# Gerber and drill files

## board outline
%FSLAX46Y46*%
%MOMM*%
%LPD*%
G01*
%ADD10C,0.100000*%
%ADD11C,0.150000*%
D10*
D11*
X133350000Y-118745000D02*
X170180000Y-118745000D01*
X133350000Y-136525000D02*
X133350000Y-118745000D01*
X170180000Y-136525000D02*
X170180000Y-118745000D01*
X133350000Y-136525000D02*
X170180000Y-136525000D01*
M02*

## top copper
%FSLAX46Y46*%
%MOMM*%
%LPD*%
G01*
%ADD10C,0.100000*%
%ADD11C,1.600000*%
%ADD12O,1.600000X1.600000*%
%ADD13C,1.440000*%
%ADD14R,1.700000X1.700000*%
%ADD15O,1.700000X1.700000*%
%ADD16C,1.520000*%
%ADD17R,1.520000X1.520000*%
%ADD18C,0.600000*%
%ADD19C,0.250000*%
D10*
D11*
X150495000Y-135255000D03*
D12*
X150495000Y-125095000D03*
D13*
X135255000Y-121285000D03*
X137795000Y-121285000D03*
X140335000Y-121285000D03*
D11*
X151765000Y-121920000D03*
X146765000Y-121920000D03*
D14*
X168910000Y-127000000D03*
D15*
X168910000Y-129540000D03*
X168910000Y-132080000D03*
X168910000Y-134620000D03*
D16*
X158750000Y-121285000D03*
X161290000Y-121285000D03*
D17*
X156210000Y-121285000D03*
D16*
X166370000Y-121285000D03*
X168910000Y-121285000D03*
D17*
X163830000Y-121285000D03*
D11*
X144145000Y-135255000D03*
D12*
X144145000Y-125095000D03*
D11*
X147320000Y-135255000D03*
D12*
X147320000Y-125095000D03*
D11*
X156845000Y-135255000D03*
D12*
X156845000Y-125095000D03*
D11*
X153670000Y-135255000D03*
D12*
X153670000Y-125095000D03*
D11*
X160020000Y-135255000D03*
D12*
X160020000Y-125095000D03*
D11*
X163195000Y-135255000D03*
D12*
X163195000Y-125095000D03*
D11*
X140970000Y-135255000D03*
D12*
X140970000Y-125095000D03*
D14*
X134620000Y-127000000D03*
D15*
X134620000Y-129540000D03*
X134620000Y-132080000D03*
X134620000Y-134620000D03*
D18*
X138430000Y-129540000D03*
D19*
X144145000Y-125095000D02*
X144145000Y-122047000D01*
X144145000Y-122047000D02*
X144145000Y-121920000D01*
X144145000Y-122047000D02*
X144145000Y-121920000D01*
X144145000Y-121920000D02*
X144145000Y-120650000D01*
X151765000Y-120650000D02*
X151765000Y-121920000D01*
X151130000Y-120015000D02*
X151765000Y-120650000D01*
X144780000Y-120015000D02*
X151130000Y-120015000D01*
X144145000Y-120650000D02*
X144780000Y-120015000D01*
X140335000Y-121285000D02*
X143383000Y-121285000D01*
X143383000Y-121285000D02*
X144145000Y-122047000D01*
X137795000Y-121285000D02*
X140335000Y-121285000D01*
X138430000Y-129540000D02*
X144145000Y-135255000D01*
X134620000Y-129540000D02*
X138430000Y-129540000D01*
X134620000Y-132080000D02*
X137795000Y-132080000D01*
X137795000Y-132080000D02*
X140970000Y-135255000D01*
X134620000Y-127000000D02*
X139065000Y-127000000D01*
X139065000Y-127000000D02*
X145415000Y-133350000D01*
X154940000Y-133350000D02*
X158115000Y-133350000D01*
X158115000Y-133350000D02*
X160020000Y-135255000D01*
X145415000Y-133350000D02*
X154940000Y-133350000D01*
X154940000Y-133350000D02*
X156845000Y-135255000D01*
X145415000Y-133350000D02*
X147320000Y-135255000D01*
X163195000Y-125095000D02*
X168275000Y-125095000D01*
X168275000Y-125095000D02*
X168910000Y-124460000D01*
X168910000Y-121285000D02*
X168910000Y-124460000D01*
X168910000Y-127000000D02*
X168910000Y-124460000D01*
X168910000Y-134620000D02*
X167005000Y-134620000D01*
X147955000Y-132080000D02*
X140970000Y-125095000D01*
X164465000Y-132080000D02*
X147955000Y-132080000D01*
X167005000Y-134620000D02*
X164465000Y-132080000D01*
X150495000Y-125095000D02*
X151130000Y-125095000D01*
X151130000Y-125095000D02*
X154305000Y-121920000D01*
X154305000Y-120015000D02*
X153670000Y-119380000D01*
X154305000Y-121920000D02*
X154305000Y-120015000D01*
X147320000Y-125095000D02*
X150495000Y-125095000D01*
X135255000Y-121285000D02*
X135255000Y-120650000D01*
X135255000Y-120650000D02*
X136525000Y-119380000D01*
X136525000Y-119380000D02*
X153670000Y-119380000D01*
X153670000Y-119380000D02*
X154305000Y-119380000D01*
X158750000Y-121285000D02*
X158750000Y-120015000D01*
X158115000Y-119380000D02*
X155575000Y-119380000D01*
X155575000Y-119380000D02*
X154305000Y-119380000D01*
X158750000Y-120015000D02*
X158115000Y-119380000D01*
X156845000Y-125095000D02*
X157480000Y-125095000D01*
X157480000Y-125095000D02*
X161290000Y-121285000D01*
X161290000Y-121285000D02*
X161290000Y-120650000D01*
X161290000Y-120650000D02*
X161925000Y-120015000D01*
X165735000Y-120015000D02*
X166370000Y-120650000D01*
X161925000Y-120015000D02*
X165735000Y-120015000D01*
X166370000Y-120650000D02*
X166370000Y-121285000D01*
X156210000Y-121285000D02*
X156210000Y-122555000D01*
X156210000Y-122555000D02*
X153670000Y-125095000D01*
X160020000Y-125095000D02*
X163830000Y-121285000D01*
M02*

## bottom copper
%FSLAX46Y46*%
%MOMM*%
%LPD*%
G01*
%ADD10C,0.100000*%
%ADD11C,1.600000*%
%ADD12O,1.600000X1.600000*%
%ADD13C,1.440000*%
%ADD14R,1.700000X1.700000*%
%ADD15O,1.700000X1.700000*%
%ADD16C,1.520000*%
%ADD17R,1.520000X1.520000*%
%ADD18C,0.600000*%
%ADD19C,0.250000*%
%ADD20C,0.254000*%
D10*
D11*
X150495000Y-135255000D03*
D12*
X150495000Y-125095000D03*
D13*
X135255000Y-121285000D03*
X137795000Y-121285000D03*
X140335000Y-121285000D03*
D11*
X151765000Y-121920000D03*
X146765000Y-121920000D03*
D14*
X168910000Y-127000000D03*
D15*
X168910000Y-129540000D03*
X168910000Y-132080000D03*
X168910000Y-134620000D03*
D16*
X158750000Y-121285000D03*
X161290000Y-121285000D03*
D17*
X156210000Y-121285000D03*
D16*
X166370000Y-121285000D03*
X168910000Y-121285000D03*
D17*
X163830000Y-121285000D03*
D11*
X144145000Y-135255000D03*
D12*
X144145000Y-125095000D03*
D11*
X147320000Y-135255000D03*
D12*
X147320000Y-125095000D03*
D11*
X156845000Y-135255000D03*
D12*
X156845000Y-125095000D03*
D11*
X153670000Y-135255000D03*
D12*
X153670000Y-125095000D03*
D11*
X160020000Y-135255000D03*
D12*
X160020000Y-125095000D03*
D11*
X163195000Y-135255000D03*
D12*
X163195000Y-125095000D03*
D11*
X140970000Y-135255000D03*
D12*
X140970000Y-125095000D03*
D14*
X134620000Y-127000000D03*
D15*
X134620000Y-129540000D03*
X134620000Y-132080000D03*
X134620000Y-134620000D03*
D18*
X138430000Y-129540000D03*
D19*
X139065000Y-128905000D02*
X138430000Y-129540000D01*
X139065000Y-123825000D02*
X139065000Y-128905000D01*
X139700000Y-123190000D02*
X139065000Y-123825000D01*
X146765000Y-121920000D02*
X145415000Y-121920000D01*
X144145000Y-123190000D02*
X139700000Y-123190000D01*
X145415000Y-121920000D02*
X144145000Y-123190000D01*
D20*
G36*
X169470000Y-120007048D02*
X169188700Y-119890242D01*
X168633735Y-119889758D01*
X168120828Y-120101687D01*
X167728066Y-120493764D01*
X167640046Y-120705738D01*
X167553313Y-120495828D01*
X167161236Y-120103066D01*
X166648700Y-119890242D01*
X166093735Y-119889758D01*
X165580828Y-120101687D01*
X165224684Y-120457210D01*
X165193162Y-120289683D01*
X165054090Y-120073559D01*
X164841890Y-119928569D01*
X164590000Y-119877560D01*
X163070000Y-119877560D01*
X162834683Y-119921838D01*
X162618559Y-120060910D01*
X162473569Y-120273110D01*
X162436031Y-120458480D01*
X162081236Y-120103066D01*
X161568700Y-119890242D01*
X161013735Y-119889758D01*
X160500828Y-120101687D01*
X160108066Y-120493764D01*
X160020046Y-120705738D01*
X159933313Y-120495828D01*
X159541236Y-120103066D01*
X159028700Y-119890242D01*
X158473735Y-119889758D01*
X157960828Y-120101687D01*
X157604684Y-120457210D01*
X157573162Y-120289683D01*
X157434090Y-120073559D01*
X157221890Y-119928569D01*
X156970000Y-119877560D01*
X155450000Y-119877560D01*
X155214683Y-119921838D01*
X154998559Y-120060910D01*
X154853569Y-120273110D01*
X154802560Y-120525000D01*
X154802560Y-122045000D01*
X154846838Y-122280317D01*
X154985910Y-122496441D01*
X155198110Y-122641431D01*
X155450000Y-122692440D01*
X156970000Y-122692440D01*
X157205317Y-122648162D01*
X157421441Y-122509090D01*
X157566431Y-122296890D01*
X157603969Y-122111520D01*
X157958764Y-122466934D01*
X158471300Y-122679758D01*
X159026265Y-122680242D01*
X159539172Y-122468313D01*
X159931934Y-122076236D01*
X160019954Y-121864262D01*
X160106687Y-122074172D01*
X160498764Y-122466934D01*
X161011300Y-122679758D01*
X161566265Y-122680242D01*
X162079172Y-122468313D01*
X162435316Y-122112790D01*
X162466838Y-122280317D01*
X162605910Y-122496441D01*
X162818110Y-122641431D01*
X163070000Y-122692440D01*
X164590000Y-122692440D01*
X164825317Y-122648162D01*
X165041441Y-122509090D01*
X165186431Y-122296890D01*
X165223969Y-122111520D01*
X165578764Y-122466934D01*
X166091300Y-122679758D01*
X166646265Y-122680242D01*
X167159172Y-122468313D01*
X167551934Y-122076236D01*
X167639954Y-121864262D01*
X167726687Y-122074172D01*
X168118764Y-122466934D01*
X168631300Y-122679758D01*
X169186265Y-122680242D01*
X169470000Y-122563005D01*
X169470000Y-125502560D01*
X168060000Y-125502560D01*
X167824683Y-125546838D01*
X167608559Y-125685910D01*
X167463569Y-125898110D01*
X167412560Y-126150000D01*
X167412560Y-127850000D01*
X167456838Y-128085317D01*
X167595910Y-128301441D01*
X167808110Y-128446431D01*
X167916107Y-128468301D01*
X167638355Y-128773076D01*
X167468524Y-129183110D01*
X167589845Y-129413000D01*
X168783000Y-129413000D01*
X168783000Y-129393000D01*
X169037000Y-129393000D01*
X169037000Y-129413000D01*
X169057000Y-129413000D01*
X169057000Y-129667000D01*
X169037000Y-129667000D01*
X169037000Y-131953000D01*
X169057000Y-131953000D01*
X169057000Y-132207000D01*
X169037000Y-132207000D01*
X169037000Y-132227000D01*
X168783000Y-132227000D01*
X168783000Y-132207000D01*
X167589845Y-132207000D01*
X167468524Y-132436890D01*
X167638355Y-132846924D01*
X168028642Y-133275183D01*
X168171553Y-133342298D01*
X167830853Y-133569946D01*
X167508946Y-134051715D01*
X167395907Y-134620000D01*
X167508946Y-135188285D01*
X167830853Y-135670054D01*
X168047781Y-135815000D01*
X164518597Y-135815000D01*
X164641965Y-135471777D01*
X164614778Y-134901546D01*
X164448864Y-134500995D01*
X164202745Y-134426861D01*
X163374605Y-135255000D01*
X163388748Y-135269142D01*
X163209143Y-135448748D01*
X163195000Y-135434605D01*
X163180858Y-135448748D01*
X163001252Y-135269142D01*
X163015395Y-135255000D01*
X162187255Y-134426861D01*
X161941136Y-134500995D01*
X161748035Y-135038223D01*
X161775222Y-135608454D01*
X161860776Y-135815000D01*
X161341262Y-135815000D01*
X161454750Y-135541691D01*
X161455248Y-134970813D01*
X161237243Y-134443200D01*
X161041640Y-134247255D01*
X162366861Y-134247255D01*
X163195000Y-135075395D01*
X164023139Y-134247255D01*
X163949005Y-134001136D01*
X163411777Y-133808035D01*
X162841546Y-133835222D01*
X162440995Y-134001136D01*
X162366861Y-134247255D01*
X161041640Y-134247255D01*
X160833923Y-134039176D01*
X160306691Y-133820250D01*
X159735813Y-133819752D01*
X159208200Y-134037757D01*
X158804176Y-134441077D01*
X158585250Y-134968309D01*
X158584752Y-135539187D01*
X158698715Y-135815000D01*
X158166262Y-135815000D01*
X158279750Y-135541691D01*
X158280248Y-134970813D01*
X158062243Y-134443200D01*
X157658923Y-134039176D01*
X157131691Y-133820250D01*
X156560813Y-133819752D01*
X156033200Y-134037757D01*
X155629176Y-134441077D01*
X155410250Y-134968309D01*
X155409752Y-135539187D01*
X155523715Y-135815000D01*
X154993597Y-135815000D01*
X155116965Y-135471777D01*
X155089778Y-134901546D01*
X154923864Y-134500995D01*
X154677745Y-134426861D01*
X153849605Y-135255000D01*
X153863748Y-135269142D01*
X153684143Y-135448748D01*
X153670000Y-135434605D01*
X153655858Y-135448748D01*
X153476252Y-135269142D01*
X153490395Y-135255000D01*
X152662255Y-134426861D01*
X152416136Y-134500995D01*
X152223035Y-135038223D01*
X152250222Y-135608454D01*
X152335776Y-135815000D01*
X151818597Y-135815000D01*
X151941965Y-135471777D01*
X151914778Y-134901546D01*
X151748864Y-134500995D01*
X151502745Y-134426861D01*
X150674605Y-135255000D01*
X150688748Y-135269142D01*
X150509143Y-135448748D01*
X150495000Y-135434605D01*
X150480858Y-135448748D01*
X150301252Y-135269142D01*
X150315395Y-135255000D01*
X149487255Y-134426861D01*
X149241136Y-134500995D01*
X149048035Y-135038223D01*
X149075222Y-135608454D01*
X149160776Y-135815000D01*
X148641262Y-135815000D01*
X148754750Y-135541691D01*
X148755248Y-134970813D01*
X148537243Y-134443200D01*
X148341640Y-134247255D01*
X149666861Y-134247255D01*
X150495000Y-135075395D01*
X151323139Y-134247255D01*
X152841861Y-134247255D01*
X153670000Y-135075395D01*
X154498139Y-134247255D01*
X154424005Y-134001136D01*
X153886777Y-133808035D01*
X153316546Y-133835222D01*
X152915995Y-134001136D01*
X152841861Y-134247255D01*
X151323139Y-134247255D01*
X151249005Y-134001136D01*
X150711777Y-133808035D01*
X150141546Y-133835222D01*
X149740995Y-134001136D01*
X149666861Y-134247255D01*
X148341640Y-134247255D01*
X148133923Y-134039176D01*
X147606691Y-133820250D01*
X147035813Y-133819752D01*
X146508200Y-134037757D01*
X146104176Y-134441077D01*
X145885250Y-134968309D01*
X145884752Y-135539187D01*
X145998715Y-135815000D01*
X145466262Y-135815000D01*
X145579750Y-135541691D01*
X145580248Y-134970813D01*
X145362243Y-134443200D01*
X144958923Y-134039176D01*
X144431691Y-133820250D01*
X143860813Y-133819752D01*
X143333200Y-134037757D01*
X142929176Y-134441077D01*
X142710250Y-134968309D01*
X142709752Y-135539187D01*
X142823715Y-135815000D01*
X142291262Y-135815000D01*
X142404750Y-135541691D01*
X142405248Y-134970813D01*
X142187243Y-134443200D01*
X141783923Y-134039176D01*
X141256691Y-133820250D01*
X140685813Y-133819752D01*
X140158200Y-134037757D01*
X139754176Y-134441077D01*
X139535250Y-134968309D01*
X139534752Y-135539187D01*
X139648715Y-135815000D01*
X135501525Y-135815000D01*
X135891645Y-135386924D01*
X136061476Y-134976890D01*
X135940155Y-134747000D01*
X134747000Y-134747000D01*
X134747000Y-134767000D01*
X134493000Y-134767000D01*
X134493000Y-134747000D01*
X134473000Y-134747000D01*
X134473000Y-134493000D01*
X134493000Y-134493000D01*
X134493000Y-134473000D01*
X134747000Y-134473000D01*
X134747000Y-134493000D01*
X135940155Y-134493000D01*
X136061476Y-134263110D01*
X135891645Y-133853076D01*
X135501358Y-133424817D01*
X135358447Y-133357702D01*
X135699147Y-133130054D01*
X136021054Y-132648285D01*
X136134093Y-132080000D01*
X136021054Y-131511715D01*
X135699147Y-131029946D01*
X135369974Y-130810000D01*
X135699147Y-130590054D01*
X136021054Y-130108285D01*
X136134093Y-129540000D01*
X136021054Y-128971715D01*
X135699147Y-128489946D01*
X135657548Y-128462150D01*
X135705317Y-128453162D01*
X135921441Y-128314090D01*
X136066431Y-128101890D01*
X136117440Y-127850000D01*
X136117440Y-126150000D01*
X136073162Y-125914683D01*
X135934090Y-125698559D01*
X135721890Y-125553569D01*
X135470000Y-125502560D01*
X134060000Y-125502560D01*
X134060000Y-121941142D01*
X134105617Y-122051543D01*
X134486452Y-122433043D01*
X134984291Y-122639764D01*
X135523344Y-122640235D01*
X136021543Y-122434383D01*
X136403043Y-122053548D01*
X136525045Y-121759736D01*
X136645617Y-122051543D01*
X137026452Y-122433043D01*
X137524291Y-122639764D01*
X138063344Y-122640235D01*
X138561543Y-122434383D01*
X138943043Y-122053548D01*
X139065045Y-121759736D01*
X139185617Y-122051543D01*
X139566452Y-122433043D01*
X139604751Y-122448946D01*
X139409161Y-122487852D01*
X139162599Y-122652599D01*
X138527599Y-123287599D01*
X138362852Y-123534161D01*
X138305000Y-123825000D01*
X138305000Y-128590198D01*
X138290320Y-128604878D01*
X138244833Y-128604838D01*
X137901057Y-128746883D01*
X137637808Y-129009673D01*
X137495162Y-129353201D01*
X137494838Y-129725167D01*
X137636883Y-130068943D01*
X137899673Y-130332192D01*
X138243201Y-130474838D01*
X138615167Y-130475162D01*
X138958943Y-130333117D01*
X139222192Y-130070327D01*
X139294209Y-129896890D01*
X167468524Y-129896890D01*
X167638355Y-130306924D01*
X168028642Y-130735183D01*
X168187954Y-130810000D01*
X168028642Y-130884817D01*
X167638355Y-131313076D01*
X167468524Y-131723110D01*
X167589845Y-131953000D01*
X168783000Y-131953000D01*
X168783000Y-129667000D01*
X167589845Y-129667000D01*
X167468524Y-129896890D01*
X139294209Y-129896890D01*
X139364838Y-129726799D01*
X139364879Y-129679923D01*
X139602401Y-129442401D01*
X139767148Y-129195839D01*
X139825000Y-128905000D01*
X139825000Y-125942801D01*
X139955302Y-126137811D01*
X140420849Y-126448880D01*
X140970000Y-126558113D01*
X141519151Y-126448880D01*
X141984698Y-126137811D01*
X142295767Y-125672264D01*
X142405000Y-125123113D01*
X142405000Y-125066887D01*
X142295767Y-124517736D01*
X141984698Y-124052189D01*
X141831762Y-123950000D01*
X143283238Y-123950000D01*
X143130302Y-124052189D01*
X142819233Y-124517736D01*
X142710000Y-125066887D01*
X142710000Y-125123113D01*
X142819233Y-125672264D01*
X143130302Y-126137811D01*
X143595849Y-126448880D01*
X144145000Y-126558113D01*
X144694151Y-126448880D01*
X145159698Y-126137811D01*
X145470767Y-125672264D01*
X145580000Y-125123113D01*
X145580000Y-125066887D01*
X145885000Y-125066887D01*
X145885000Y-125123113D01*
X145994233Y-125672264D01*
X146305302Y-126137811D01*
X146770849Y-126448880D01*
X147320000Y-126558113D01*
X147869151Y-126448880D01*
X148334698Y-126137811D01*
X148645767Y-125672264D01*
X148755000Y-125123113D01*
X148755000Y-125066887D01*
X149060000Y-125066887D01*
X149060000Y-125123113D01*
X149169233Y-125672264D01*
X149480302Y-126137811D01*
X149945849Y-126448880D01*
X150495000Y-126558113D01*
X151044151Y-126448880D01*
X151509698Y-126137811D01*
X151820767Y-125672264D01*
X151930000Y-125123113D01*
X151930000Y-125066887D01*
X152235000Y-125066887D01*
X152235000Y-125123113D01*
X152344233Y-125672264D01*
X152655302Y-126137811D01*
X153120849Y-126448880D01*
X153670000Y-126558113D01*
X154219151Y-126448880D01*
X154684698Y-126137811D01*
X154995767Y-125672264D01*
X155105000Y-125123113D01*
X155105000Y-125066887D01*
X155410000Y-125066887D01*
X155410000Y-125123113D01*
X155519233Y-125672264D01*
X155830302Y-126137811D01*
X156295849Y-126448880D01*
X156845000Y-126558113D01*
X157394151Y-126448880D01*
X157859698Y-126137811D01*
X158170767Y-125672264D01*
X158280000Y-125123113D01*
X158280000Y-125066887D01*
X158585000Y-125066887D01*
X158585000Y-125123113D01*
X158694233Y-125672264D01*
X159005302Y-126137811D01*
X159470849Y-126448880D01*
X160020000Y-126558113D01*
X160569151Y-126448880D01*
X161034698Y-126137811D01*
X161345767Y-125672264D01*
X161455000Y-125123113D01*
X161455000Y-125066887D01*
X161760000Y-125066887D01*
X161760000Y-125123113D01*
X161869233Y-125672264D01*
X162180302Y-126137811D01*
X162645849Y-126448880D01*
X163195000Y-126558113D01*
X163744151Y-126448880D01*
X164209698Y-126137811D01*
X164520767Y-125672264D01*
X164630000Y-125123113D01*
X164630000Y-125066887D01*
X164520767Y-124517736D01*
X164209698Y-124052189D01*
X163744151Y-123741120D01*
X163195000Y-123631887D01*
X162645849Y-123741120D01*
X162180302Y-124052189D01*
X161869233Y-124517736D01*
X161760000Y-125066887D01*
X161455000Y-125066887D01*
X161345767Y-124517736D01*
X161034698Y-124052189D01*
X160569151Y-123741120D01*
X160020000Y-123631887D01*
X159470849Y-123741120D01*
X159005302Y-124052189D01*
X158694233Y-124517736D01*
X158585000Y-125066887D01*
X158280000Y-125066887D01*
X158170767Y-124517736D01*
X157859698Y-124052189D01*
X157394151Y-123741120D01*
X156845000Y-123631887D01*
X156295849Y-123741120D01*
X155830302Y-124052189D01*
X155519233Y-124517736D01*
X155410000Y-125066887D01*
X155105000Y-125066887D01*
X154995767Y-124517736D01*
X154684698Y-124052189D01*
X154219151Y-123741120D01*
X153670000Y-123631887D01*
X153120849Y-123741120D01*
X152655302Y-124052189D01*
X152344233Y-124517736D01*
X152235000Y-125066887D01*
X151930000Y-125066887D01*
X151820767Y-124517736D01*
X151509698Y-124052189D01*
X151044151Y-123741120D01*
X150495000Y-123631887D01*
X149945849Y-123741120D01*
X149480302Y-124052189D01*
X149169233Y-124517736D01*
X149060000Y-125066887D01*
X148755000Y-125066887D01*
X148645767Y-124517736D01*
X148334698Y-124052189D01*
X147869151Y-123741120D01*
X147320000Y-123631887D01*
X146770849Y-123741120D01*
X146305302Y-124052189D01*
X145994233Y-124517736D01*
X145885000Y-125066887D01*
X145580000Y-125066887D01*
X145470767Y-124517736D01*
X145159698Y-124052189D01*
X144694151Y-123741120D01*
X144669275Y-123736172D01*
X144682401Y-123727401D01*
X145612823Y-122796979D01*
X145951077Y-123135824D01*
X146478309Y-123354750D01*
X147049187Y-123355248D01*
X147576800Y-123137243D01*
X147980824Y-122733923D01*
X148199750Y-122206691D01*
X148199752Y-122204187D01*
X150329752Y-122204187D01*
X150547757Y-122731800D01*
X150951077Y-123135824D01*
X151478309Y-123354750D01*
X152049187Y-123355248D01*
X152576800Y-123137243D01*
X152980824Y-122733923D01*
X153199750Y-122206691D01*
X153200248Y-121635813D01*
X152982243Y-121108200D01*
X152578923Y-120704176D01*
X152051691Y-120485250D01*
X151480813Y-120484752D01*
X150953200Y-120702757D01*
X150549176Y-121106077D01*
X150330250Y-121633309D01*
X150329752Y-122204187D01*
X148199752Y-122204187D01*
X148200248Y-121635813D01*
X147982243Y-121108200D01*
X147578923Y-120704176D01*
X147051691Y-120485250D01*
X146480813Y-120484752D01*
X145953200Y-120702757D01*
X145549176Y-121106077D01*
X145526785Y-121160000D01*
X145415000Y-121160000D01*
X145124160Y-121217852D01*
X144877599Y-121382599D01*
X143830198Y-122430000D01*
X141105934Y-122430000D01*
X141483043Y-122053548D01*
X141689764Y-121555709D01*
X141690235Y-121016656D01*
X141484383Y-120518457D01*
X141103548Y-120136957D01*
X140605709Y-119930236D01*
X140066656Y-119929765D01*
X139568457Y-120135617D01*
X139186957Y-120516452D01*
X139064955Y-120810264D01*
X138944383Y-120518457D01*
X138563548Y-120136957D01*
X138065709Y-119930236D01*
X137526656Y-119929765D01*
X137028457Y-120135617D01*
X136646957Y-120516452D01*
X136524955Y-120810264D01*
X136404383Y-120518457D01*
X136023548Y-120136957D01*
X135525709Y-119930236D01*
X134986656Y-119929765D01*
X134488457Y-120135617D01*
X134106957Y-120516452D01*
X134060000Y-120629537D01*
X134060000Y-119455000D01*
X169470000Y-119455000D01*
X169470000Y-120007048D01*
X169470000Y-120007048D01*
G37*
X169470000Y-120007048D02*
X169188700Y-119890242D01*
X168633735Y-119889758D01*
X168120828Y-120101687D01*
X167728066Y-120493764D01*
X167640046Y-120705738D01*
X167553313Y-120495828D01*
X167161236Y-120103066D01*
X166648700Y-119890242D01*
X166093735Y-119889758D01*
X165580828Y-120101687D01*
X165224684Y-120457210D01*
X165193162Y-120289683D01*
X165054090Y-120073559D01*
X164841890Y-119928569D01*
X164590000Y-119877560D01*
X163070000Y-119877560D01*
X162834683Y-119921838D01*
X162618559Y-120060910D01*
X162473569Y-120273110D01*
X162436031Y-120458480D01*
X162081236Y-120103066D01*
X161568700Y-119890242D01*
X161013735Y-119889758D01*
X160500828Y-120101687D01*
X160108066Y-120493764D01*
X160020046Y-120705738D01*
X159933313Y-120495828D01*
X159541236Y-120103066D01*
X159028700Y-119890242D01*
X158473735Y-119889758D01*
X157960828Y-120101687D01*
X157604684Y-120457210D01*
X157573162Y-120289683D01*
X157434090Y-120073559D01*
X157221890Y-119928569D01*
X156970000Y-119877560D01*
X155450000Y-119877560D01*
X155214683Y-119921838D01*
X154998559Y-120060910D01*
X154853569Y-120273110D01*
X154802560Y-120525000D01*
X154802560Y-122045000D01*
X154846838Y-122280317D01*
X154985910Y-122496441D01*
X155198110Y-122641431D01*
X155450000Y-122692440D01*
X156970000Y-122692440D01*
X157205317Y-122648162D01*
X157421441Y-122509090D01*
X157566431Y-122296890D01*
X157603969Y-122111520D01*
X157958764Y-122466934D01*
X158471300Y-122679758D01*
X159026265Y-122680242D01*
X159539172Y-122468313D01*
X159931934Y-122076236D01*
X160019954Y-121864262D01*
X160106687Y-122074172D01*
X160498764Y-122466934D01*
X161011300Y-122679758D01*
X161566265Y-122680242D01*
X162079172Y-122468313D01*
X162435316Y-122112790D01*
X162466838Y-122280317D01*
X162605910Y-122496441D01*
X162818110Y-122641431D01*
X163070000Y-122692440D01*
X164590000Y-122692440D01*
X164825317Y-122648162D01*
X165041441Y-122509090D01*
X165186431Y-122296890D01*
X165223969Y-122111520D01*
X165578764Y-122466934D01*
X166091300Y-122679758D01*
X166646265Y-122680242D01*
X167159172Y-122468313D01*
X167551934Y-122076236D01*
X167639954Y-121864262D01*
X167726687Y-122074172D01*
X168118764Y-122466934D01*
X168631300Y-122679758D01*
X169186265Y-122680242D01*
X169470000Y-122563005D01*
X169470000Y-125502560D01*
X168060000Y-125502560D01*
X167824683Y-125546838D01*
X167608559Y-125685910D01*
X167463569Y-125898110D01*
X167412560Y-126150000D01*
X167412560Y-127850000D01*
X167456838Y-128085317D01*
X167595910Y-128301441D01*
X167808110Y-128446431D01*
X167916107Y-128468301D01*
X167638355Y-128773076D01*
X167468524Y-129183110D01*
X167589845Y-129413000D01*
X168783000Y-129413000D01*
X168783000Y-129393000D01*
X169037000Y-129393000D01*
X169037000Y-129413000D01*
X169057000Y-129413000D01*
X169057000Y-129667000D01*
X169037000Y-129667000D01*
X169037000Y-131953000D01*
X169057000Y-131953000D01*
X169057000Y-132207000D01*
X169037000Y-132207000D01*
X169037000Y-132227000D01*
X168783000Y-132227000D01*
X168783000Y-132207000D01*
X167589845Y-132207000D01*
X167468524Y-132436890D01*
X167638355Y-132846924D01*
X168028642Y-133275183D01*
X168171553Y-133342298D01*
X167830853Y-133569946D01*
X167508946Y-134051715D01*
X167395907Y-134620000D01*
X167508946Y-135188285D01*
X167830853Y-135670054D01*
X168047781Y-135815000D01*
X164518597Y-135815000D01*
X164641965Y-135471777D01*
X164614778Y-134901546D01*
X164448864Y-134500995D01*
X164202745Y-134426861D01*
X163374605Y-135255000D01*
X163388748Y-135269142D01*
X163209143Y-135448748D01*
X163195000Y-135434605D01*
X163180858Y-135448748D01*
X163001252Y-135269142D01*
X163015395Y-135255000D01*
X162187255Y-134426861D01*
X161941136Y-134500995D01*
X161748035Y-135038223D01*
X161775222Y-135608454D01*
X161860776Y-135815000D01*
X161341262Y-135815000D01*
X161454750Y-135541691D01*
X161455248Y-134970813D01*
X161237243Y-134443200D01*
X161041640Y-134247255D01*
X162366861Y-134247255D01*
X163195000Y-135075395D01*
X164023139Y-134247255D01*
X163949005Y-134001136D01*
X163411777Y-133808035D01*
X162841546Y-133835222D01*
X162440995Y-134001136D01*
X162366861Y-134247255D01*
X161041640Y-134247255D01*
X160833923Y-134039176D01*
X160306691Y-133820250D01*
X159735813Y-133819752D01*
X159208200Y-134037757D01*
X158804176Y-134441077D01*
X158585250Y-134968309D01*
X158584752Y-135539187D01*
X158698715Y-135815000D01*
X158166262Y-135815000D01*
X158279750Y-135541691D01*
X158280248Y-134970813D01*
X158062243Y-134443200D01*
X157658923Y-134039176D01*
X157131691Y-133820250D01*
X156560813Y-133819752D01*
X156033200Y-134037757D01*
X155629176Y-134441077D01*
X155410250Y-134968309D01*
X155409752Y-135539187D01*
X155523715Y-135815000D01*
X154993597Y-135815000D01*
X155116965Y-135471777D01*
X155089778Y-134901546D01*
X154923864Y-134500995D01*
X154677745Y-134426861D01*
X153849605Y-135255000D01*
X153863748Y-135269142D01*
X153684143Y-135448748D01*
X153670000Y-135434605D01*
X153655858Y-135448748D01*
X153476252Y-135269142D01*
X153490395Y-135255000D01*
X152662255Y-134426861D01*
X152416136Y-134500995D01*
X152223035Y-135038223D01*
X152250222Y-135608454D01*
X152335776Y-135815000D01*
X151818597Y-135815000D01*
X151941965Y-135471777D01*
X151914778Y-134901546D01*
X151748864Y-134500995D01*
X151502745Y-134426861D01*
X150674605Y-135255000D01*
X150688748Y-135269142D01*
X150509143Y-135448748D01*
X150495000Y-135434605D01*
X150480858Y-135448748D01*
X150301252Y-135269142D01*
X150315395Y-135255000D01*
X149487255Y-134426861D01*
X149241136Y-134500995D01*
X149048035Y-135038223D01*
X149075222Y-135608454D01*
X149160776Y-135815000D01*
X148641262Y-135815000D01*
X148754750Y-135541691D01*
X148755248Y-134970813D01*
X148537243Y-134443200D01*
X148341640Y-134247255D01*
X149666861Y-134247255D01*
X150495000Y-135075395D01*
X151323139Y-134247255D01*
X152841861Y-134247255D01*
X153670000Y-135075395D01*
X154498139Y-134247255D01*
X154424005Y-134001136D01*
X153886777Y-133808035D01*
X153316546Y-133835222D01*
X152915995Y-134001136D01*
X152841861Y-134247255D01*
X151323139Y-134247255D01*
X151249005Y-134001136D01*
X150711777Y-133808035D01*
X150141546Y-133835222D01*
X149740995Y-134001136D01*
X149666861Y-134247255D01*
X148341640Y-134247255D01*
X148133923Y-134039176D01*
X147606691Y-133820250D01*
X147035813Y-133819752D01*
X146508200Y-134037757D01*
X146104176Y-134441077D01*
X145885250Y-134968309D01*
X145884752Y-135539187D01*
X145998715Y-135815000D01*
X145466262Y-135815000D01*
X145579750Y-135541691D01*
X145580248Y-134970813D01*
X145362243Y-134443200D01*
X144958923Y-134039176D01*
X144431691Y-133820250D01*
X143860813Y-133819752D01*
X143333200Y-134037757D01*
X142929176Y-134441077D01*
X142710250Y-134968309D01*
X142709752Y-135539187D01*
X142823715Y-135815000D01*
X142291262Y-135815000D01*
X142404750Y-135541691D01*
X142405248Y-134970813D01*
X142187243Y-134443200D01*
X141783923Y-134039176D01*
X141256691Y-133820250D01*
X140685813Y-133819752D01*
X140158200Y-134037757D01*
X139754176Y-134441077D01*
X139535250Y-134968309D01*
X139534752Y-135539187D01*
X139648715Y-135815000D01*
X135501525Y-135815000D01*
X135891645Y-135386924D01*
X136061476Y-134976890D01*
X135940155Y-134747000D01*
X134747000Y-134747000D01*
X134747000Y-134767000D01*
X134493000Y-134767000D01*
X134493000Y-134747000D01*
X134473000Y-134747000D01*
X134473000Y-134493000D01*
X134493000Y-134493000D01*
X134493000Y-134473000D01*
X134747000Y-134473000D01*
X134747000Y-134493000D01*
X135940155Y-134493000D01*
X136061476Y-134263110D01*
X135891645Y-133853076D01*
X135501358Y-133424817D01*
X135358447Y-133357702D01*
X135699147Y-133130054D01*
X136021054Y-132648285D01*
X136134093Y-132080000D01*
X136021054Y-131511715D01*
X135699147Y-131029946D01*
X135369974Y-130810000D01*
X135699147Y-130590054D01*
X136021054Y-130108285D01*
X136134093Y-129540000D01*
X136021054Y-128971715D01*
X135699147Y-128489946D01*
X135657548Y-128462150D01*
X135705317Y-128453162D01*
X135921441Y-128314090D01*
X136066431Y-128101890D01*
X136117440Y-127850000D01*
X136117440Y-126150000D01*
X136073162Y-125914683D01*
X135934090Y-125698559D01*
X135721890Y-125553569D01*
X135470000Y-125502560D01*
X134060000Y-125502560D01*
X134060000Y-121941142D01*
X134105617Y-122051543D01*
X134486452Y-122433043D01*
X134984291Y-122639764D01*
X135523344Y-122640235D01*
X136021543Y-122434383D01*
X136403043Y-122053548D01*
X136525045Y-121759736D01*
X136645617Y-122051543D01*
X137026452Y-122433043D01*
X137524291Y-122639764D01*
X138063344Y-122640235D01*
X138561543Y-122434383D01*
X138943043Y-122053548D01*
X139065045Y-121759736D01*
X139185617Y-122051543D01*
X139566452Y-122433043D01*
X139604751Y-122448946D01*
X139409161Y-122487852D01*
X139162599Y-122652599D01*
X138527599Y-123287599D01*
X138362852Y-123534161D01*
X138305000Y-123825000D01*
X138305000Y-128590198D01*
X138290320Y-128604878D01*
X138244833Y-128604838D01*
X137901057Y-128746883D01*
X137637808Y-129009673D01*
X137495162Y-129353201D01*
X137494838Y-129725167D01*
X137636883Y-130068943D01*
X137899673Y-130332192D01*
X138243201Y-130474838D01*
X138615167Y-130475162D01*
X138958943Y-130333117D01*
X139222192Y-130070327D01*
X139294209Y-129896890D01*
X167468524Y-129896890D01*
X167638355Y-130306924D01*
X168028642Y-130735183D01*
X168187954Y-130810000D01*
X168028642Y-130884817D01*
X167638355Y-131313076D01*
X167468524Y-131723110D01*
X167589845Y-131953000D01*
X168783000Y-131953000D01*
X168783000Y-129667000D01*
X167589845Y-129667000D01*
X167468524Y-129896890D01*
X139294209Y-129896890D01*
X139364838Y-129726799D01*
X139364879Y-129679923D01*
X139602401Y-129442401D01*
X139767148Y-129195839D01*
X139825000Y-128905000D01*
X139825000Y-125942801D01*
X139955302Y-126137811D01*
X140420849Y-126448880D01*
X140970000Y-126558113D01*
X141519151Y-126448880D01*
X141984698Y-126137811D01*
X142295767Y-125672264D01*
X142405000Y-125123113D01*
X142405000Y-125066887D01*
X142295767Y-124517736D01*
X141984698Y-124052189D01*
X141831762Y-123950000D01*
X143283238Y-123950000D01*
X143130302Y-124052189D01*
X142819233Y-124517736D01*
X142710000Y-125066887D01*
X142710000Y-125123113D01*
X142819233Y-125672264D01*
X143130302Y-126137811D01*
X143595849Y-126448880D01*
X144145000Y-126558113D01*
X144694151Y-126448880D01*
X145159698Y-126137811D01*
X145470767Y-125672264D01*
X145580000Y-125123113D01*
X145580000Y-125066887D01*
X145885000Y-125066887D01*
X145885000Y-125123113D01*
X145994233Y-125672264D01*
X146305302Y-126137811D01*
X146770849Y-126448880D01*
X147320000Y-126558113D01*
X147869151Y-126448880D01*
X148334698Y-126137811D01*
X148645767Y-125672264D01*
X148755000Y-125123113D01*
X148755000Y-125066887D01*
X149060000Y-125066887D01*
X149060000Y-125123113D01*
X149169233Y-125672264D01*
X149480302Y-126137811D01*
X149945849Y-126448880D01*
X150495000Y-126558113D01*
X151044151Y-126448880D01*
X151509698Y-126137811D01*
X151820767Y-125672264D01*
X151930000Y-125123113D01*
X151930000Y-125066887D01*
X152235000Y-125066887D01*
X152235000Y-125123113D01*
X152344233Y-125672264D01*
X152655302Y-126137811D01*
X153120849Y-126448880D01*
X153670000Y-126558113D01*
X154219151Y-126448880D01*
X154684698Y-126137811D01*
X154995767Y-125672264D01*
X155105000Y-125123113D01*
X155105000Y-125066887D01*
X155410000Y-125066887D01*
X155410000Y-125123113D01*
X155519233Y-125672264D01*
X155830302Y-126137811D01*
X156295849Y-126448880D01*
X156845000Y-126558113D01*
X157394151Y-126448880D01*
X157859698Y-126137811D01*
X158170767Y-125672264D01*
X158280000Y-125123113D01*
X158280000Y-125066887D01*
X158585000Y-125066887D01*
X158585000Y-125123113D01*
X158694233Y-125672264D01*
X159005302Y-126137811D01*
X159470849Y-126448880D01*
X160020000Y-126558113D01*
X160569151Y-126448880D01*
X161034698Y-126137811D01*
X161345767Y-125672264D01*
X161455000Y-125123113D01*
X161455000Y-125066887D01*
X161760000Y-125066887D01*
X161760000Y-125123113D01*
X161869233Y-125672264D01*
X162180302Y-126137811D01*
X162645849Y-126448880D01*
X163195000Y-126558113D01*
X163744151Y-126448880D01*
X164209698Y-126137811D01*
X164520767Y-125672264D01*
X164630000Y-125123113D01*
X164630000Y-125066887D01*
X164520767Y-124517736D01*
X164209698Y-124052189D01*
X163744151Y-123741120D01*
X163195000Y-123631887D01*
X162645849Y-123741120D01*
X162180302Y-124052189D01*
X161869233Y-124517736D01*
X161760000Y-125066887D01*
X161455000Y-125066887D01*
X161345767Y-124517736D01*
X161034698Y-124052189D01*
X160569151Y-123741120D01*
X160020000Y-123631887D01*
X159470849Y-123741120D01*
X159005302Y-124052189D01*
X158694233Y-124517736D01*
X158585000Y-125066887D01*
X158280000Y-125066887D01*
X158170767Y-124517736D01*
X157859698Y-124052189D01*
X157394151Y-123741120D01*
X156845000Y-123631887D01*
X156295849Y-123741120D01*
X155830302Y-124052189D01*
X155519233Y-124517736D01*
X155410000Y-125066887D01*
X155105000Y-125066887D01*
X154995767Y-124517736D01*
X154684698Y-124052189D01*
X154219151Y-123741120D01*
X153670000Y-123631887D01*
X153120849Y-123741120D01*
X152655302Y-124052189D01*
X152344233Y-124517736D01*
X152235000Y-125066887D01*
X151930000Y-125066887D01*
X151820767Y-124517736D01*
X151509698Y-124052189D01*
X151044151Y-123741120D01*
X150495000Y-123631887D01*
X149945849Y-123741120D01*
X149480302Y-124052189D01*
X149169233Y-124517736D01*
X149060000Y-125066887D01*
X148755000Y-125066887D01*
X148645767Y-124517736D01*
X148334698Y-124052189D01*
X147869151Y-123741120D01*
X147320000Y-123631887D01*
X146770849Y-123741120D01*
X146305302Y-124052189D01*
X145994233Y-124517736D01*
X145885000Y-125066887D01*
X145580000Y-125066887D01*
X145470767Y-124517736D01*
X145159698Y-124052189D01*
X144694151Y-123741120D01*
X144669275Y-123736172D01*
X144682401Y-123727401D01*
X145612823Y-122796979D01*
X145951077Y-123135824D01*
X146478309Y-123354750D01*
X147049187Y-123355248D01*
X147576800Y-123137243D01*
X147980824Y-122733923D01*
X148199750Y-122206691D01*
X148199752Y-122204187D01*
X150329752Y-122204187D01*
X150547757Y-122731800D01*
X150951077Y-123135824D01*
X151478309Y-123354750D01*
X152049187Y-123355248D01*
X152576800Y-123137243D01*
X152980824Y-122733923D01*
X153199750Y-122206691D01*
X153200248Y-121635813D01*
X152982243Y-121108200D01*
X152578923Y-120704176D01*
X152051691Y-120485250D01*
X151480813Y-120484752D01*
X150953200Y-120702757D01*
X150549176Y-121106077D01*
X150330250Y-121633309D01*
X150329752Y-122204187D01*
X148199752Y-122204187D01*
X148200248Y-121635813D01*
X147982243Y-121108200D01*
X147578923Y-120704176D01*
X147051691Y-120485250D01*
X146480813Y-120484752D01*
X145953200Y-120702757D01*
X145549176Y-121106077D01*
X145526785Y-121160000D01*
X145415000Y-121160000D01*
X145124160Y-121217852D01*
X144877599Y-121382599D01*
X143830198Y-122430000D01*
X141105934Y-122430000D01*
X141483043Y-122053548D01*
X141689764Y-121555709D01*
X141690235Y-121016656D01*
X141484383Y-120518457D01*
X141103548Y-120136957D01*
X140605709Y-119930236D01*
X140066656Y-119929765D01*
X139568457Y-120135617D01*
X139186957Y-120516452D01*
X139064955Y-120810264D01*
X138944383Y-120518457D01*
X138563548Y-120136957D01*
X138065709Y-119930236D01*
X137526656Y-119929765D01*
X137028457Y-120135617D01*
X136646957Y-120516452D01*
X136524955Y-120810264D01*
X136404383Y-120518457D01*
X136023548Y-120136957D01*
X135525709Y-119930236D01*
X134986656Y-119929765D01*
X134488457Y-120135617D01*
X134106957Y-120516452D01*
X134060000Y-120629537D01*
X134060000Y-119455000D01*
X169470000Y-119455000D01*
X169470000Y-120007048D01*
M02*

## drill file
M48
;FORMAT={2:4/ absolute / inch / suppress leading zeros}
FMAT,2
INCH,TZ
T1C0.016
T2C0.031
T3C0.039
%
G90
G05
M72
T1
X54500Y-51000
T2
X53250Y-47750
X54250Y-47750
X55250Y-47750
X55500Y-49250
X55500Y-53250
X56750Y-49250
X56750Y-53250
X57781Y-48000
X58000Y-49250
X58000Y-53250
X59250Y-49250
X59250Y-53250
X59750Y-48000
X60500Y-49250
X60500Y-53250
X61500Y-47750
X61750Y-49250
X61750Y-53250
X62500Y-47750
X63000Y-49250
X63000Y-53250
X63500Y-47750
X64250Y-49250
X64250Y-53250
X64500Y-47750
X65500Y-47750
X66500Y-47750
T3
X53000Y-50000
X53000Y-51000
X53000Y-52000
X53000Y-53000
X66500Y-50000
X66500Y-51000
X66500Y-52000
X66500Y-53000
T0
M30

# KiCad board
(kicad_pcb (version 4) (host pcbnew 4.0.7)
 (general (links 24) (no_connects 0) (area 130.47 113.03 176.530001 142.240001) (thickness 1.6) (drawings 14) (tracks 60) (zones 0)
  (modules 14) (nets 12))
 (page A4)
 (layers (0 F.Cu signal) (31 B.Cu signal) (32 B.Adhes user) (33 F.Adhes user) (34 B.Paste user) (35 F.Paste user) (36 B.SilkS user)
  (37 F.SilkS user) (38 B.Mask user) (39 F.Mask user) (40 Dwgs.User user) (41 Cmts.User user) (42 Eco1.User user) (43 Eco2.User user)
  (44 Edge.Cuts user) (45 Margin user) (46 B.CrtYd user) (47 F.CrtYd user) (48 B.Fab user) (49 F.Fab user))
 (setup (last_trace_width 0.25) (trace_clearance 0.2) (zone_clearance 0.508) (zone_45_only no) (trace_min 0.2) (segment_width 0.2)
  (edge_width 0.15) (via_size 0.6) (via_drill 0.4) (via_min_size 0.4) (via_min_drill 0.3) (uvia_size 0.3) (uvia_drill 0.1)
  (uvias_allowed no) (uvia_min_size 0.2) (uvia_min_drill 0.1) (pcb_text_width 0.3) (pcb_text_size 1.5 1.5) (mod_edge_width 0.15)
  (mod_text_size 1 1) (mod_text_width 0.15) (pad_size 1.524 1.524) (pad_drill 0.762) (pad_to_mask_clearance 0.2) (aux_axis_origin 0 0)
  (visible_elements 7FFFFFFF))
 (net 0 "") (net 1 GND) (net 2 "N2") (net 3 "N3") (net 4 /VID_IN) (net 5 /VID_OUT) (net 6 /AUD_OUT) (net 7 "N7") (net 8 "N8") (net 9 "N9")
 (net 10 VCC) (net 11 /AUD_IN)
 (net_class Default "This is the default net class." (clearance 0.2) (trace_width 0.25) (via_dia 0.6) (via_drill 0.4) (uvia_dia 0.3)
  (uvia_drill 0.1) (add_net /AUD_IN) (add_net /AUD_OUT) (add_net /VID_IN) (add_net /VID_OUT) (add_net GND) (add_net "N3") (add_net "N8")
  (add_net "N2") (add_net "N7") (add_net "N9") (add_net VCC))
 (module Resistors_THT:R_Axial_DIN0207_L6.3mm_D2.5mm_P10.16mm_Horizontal (layer F.Cu) (at 150.495 135.255 90)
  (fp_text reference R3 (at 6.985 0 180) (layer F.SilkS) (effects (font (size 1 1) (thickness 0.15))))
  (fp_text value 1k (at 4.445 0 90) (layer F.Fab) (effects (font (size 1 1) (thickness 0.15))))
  (pad 1 thru_hole circle (at 0 0 90) (size 1.6 1.6) (drill 0.8) (layers *.Cu *.Mask) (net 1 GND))
  (pad 2 thru_hole oval (at 10.16 0 90) (size 1.6 1.6) (drill 0.8) (layers *.Cu *.Mask) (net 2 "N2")))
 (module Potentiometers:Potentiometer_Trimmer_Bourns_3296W (layer F.Cu) (at 135.255 121.285 180)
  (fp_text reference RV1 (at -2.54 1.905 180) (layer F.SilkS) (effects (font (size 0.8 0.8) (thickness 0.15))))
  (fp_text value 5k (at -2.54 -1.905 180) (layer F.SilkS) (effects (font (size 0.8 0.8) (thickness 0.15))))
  (pad 1 thru_hole circle (at 0 0 180) (size 1.44 1.44) (drill 0.8) (layers *.Cu *.Mask) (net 2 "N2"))
  (pad 2 thru_hole circle (at -2.54 0 180) (size 1.44 1.44) (drill 0.8) (layers *.Cu *.Mask) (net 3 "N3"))
  (pad 3 thru_hole circle (at -5.08 0 180) (size 1.44 1.44) (drill 0.8) (layers *.Cu *.Mask) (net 3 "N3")))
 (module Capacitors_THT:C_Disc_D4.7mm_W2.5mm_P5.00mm (layer F.Cu) (at 151.765 121.92 180)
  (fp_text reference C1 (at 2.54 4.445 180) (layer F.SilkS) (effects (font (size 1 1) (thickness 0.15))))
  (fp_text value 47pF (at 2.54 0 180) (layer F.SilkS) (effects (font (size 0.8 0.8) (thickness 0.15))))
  (pad 1 thru_hole circle (at 0 0 180) (size 1.6 1.6) (drill 0.8) (layers *.Cu *.Mask) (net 3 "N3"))
  (pad 2 thru_hole circle (at 5 0 180) (size 1.6 1.6) (drill 0.8) (layers *.Cu *.Mask) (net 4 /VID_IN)))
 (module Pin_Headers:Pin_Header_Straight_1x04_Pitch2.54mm (layer F.Cu) (at 168.91 127)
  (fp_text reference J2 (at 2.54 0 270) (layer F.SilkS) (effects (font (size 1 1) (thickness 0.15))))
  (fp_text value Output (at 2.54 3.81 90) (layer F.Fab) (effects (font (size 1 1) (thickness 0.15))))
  (pad 1 thru_hole rect (at 0 0) (size 1.7 1.7) (drill 1) (layers *.Cu *.Mask) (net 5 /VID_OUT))
  (pad 2 thru_hole oval (at 0 2.54) (size 1.7 1.7) (drill 1) (layers *.Cu *.Mask) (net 1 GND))
  (pad 3 thru_hole oval (at 0 5.08) (size 1.7 1.7) (drill 1) (layers *.Cu *.Mask) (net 1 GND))
  (pad 4 thru_hole oval (at 0 7.62) (size 1.7 1.7) (drill 1) (layers *.Cu *.Mask) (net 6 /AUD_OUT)))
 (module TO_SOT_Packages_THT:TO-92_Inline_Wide (layer F.Cu) (at 156.21 121.285)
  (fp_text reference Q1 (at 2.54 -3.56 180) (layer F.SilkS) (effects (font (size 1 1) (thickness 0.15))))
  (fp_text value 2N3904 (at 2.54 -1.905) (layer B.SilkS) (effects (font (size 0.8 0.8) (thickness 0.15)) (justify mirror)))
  (pad 2 thru_hole circle (at 2.54 0 90) (size 1.52 1.52) (drill 0.8) (layers *.Cu *.Mask) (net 2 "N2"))
  (pad 3 thru_hole circle (at 5.08 0 90) (size 1.52 1.52) (drill 0.8) (layers *.Cu *.Mask) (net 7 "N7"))
  (pad 1 thru_hole rect (at 0 0 90) (size 1.52 1.52) (drill 0.8) (layers *.Cu *.Mask) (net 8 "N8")))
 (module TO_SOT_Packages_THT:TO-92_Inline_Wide (layer F.Cu) (at 163.83 121.285)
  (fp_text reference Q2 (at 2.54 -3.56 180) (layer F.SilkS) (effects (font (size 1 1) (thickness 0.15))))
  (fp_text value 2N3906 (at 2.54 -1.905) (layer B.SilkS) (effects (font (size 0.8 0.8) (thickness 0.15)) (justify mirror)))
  (pad 2 thru_hole circle (at 2.54 0 90) (size 1.52 1.52) (drill 0.8) (layers *.Cu *.Mask) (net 7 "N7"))
  (pad 3 thru_hole circle (at 5.08 0 90) (size 1.52 1.52) (drill 0.8) (layers *.Cu *.Mask) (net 5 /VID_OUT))
  (pad 1 thru_hole rect (at 0 0 90) (size 1.52 1.52) (drill 0.8) (layers *.Cu *.Mask) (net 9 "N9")))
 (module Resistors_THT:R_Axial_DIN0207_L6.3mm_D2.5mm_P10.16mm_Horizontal (layer F.Cu) (at 144.145 135.255 90)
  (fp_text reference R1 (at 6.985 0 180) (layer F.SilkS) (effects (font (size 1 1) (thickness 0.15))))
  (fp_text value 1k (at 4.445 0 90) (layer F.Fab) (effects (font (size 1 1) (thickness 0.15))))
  (pad 1 thru_hole circle (at 0 0 90) (size 1.6 1.6) (drill 0.8) (layers *.Cu *.Mask) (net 4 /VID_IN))
  (pad 2 thru_hole oval (at 10.16 0 90) (size 1.6 1.6) (drill 0.8) (layers *.Cu *.Mask) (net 3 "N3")))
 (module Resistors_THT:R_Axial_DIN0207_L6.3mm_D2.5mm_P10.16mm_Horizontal (layer F.Cu) (at 147.32 135.255 90)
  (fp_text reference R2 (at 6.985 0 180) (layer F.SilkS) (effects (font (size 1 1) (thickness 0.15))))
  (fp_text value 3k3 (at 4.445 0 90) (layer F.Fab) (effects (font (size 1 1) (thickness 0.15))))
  (pad 1 thru_hole circle (at 0 0 90) (size 1.6 1.6) (drill 0.8) (layers *.Cu *.Mask) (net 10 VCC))
  (pad 2 thru_hole oval (at 10.16 0 90) (size 1.6 1.6) (drill 0.8) (layers *.Cu *.Mask) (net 2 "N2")))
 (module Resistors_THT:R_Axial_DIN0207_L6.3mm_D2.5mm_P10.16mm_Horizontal (layer F.Cu) (at 156.845 135.255 90)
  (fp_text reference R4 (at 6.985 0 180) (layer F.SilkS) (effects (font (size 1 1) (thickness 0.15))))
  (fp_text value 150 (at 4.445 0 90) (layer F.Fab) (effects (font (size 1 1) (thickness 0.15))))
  (pad 1 thru_hole circle (at 0 0 90) (size 1.6 1.6) (drill 0.8) (layers *.Cu *.Mask) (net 10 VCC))
  (pad 2 thru_hole oval (at 10.16 0 90) (size 1.6 1.6) (drill 0.8) (layers *.Cu *.Mask) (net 7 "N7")))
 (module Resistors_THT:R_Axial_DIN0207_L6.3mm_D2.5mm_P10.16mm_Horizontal (layer F.Cu) (at 153.67 135.255 90)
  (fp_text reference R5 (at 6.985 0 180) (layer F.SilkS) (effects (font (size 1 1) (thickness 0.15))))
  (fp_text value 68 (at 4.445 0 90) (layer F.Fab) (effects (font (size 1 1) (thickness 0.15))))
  (pad 1 thru_hole circle (at 0 0 90) (size 1.6 1.6) (drill 0.8) (layers *.Cu *.Mask) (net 1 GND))
  (pad 2 thru_hole oval (at 10.16 0 90) (size 1.6 1.6) (drill 0.8) (layers *.Cu *.Mask) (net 8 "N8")))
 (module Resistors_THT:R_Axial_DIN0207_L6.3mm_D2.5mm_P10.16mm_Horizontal (layer F.Cu) (at 160.02 135.255 90)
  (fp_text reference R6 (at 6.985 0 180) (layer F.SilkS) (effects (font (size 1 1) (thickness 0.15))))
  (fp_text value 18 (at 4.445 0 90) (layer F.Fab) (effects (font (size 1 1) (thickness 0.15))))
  (pad 1 thru_hole circle (at 0 0 90) (size 1.6 1.6) (drill 0.8) (layers *.Cu *.Mask) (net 10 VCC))
  (pad 2 thru_hole oval (at 10.16 0 90) (size 1.6 1.6) (drill 0.8) (layers *.Cu *.Mask) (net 9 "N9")))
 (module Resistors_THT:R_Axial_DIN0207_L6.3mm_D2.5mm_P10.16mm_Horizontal (layer F.Cu) (at 163.195 135.255 90)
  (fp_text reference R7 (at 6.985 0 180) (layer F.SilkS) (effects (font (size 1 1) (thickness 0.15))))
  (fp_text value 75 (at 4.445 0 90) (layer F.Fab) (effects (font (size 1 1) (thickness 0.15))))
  (pad 1 thru_hole circle (at 0 0 90) (size 1.6 1.6) (drill 0.8) (layers *.Cu *.Mask) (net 1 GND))
  (pad 2 thru_hole oval (at 10.16 0 90) (size 1.6 1.6) (drill 0.8) (layers *.Cu *.Mask) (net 5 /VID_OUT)))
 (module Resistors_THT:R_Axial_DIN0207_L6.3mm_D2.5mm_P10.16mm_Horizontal (layer F.Cu) (at 140.97 135.255 90)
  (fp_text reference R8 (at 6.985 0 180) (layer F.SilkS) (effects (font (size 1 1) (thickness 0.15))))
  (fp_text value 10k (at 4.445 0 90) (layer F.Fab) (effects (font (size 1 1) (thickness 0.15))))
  (pad 1 thru_hole circle (at 0 0 90) (size 1.6 1.6) (drill 0.8) (layers *.Cu *.Mask) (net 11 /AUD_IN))
  (pad 2 thru_hole oval (at 10.16 0 90) (size 1.6 1.6) (drill 0.8) (layers *.Cu *.Mask) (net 6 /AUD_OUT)))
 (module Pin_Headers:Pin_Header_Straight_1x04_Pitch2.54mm (layer F.Cu) (at 134.62 127)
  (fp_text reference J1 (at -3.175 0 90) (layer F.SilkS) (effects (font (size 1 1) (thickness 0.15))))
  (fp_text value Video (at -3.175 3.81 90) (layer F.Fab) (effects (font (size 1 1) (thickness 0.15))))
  (pad 1 thru_hole rect (at 0 0) (size 1.7 1.7) (drill 1) (layers *.Cu *.Mask) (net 10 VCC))
  (pad 2 thru_hole oval (at 0 2.54) (size 1.7 1.7) (drill 1) (layers *.Cu *.Mask) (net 4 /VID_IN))
  (pad 3 thru_hole oval (at 0 5.08) (size 1.7 1.7) (drill 1) (layers *.Cu *.Mask) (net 11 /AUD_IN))
  (pad 4 thru_hole oval (at 0 7.62) (size 1.7 1.7) (drill 1) (layers *.Cu *.Mask) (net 1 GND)))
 (gr_line (start 133.35 118.745) (end 170.18 118.745) (angle 90) (layer Edge.Cuts) (width 0.15))
 (gr_line (start 133.35 136.525) (end 133.35 118.745) (angle 90) (layer Edge.Cuts) (width 0.15))
 (gr_line (start 170.18 136.525) (end 170.18 118.745) (angle 90) (layer Edge.Cuts) (width 0.15))
 (gr_line (start 133.35 136.525) (end 170.18 136.525) (angle 90) (layer Edge.Cuts) (width 0.15))
 (segment (start 144.145 125.095) (end 144.145 122.047) (width 0.25) (layer F.Cu) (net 3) (status 400000))
 (segment (start 144.145 122.047) (end 144.145 121.92) (width 0.25) (layer F.Cu) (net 3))
 (segment (start 144.145 122.047) (end 144.145 121.92) (width 0.25) (layer F.Cu) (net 3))
 (segment (start 144.145 121.92) (end 144.145 120.65) (width 0.25) (layer F.Cu) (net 3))
 (segment (start 151.765 120.65) (end 151.765 121.92) (width 0.25) (layer F.Cu) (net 3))
 (segment (start 151.13 120.015) (end 151.765 120.65) (width 0.25) (layer F.Cu) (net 3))
 (segment (start 144.78 120.015) (end 151.13 120.015) (width 0.25) (layer F.Cu) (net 3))
 (segment (start 144.145 120.65) (end 144.78 120.015) (width 0.25) (layer F.Cu) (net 3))
 (segment (start 140.335 121.285) (end 143.383 121.285) (width 0.25) (layer F.Cu) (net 3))
 (segment (start 143.383 121.285) (end 144.145 122.047) (width 0.25) (layer F.Cu) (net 3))
 (segment (start 137.795 121.285) (end 140.335 121.285) (width 0.25) (layer F.Cu) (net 3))
 (segment (start 138.43 129.54) (end 144.145 135.255) (width 0.25) (layer F.Cu) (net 4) (status 800000))
 (segment (start 139.065 128.905) (end 138.43 129.54) (width 0.25) (layer B.Cu) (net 4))
 (segment (start 139.065 123.825) (end 139.065 128.905) (width 0.25) (layer B.Cu) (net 4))
 (segment (start 139.7 123.19) (end 139.065 123.825) (width 0.25) (layer B.Cu) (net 4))
 (segment (start 146.765 121.92) (end 145.415 121.92) (width 0.25) (layer B.Cu) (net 4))
 (via (at 138.43 129.54) (size 0.6) (drill 0.4) (layers F.Cu B.Cu) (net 4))
 (segment (start 144.145 123.19) (end 139.7 123.19) (width 0.25) (layer B.Cu) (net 4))
 (segment (start 145.415 121.92) (end 144.145 123.19) (width 0.25) (layer B.Cu) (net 4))
 (segment (start 134.62 129.54) (end 138.43 129.54) (width 0.25) (layer F.Cu) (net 4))
 (segment (start 134.62 132.08) (end 137.795 132.08) (width 0.25) (layer F.Cu) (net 11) (status 400000))
 (segment (start 137.795 132.08) (end 140.97 135.255) (width 0.25) (layer F.Cu) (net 11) (status 800000))
 (segment (start 134.62 127) (end 139.065 127) (width 0.25) (layer F.Cu) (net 10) (status 400000))
 (segment (start 139.065 127) (end 145.415 133.35) (width 0.25) (layer F.Cu) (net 10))
 (segment (start 154.94 133.35) (end 158.115 133.35) (width 0.25) (layer F.Cu) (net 10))
 (segment (start 158.115 133.35) (end 160.02 135.255) (width 0.25) (layer F.Cu) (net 10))
 (segment (start 145.415 133.35) (end 154.94 133.35) (width 0.25) (layer F.Cu) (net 10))
 (segment (start 154.94 133.35) (end 156.845 135.255) (width 0.25) (layer F.Cu) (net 10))
 (segment (start 145.415 133.35) (end 147.32 135.255) (width 0.25) (layer F.Cu) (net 10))
 (segment (start 163.195 125.095) (end 168.275 125.095) (width 0.25) (layer F.Cu) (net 5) (status 400000))
 (segment (start 168.275 125.095) (end 168.91 124.46) (width 0.25) (layer F.Cu) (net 5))
 (segment (start 168.91 121.285) (end 168.91 124.46) (width 0.25) (layer F.Cu) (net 5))
 (segment (start 168.91 127) (end 168.91 124.46) (width 0.25) (layer F.Cu) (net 5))
 (segment (start 168.91 134.62) (end 167.005 134.62) (width 0.25) (layer F.Cu) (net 6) (status 400000))
 (segment (start 147.955 132.08) (end 140.97 125.095) (width 0.25) (layer F.Cu) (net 6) (status 800000))
 (segment (start 164.465 132.08) (end 147.955 132.08) (width 0.25) (layer F.Cu) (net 6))
 (segment (start 167.005 134.62) (end 164.465 132.08) (width 0.25) (layer F.Cu) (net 6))
 (segment (start 150.495 125.095) (end 151.13 125.095) (width 0.25) (layer F.Cu) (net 2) (status C00000))
 (segment (start 151.13 125.095) (end 154.305 121.92) (width 0.25) (layer F.Cu) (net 2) (status 400000))
 (segment (start 154.305 120.015) (end 153.67 119.38) (width 0.25) (layer F.Cu) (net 2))
 (segment (start 154.305 121.92) (end 154.305 120.015) (width 0.25) (layer F.Cu) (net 2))
 (segment (start 147.32 125.095) (end 150.495 125.095) (width 0.25) (layer F.Cu) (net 2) (status C00000))
 (segment (start 135.255 121.285) (end 135.255 120.65) (width 0.25) (layer F.Cu) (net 2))
 (segment (start 135.255 120.65) (end 136.525 119.38) (width 0.25) (layer F.Cu) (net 2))
 (segment (start 136.525 119.38) (end 153.67 119.38) (width 0.25) (layer F.Cu) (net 2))
 (segment (start 153.67 119.38) (end 154.305 119.38) (width 0.25) (layer F.Cu) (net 2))
 (segment (start 158.75 121.285) (end 158.75 120.015) (width 0.25) (layer F.Cu) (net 2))
 (segment (start 158.115 119.38) (end 155.575 119.38) (width 0.25) (layer F.Cu) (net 2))
 (segment (start 155.575 119.38) (end 154.305 119.38) (width 0.25) (layer F.Cu) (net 2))
 (segment (start 158.75 120.015) (end 158.115 119.38) (width 0.25) (layer F.Cu) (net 2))
 (segment (start 156.845 125.095) (end 157.48 125.095) (width 0.25) (layer F.Cu) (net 7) (status C00000))
 (segment (start 157.48 125.095) (end 161.29 121.285) (width 0.25) (layer F.Cu) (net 7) (status C00000))
 (segment (start 161.29 121.285) (end 161.29 120.65) (width 0.25) (layer F.Cu) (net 7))
 (segment (start 161.29 120.65) (end 161.925 120.015) (width 0.25) (layer F.Cu) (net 7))
 (segment (start 165.735 120.015) (end 166.37 120.65) (width 0.25) (layer F.Cu) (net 7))
 (segment (start 161.925 120.015) (end 165.735 120.015) (width 0.25) (layer F.Cu) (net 7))
 (segment (start 166.37 120.65) (end 166.37 121.285) (width 0.25) (layer F.Cu) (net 7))
 (segment (start 156.21 121.285) (end 156.21 122.555) (width 0.25) (layer F.Cu) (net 8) (status 400000))
 (segment (start 156.21 122.555) (end 153.67 125.095) (width 0.25) (layer F.Cu) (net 8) (status 800000))
 (segment (start 160.02 125.095) (end 163.83 121.285) (width 0.25) (layer F.Cu) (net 9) (status C00000))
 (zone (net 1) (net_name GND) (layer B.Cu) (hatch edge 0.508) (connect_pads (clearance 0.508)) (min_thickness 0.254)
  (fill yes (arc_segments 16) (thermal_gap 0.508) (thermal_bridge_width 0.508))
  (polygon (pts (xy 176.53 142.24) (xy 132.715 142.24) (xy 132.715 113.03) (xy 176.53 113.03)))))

